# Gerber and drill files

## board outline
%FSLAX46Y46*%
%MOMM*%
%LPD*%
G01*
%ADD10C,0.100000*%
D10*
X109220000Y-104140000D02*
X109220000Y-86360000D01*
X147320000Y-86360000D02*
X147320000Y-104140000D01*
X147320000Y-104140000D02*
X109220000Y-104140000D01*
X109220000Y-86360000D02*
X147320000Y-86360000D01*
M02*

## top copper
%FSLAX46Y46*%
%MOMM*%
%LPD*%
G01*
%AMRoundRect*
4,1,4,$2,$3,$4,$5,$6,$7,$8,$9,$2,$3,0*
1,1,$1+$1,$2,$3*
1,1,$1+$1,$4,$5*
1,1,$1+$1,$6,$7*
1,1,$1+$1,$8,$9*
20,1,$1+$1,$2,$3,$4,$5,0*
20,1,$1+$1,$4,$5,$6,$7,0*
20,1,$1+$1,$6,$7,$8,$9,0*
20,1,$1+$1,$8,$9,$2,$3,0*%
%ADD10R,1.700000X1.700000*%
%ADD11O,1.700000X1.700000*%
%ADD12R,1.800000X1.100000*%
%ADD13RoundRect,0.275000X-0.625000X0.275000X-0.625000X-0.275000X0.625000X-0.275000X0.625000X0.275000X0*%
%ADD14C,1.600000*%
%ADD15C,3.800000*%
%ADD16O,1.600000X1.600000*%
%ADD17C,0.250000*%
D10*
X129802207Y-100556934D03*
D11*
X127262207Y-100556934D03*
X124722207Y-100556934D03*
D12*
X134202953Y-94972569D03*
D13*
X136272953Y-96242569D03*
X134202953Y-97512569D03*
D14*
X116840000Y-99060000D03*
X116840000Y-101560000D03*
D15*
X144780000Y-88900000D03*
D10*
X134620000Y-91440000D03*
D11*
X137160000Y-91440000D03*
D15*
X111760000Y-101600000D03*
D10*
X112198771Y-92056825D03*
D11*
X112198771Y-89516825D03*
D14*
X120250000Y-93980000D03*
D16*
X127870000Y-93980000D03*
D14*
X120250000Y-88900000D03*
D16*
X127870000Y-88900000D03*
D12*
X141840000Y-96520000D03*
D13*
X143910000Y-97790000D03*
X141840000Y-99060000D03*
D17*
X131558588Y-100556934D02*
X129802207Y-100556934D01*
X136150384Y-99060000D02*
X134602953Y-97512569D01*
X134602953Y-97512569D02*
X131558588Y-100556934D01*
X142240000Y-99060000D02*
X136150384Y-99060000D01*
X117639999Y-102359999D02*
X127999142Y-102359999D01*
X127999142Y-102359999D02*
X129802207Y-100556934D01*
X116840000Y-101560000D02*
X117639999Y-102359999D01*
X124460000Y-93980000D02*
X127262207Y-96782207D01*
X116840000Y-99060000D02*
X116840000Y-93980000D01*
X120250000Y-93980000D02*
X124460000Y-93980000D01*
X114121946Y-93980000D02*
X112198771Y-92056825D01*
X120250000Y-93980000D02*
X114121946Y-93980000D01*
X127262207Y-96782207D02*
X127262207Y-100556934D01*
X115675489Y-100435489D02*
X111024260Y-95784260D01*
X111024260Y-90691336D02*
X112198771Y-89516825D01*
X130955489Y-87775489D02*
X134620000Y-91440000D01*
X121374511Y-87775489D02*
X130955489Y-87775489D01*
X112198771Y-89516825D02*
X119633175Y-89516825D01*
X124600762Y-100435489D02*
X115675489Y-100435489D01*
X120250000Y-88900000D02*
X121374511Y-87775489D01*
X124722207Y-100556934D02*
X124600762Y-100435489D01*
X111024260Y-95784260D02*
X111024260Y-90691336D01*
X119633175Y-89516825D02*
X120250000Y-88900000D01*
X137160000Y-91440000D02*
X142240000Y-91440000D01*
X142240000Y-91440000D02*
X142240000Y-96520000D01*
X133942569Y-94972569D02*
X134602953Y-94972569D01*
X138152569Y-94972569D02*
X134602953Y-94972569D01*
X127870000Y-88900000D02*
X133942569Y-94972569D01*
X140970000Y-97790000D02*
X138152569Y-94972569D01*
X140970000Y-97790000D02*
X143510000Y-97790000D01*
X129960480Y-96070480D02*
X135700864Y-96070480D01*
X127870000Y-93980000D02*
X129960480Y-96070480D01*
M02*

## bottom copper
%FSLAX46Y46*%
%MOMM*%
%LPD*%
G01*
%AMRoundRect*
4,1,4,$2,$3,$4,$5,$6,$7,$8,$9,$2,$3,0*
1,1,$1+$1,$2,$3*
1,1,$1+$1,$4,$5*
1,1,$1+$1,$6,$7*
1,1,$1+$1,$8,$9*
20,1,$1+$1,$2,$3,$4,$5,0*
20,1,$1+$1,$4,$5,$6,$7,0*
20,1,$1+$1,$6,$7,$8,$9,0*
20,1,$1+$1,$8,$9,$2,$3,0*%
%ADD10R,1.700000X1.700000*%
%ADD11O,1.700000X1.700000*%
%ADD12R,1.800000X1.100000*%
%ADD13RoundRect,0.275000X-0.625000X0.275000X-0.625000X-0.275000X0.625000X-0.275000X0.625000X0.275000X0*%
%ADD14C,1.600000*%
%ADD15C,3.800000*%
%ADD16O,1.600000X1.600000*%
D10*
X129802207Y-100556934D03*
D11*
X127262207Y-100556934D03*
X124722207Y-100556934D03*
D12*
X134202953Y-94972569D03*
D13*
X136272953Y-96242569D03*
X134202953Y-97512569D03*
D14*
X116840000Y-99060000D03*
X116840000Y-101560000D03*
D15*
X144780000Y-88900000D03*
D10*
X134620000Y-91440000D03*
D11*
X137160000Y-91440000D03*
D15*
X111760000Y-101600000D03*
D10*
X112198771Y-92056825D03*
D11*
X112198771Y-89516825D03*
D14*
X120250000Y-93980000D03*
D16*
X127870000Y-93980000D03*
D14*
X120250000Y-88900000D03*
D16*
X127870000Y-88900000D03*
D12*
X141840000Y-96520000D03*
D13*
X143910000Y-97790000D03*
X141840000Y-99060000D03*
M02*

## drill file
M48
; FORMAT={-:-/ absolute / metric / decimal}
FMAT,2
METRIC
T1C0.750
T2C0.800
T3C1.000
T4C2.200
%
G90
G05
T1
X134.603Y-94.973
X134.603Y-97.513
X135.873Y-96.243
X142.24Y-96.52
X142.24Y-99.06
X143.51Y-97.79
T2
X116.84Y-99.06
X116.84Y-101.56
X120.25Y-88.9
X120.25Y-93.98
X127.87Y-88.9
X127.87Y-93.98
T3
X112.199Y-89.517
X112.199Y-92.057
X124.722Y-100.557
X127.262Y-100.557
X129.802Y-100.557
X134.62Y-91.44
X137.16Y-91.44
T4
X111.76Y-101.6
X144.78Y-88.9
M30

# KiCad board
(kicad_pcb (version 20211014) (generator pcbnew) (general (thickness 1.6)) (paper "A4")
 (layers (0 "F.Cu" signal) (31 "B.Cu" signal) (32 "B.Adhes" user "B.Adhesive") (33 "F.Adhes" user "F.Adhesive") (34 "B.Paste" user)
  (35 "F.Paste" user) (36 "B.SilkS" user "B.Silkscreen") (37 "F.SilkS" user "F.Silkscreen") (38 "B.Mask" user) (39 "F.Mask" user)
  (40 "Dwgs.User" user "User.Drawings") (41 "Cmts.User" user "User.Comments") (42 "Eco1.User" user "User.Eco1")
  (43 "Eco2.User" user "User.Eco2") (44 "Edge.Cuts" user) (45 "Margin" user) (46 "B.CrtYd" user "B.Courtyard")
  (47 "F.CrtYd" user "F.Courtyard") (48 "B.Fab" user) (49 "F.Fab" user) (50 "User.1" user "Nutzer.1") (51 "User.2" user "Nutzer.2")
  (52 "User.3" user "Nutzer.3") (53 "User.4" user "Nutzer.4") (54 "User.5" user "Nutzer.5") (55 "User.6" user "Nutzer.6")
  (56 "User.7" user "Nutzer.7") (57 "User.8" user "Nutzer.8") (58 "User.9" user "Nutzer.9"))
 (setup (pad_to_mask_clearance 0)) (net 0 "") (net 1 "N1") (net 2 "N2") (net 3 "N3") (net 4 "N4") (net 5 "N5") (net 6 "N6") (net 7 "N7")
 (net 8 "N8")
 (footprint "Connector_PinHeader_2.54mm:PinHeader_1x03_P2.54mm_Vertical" (layer "F.Cu") (at 129.802207 100.556934 -90)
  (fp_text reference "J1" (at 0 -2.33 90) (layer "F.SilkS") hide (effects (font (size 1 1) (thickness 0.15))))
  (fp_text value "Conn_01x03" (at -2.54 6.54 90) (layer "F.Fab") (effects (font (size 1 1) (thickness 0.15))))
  (pad "1" thru_hole rect (at 0 0 270) (size 1.7 1.7) (drill 1) (layers *.Cu *.Mask) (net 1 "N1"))
  (pad "2" thru_hole oval (at 0 2.54 270) (size 1.7 1.7) (drill 1) (layers *.Cu *.Mask) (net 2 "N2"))
  (pad "3" thru_hole oval (at 0 5.08 270) (size 1.7 1.7) (drill 1) (layers *.Cu *.Mask) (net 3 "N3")))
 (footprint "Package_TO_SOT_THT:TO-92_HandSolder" (layer "F.Cu") (at 134.602953 94.972569 -90)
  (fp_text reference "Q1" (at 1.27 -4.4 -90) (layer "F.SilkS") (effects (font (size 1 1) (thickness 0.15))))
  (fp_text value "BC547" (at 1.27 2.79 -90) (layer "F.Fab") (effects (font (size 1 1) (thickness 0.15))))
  (pad "1" thru_hole rect (at 0 0 270) (size 1.1 1.8) (drill 0.75 (offset 0 0.4)) (layers *.Cu *.Mask) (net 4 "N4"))
  (pad "2" thru_hole roundrect (at 1.27 -1.27 270) (size 1.1 1.8) (drill 0.75 (offset 0 -0.4)) (layers *.Cu *.Mask) (roundrect_rratio 0.25)
   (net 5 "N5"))
  (pad "3" thru_hole roundrect (at 2.54 0 270) (size 1.1 1.8) (drill 0.75 (offset 0 0.4)) (layers *.Cu *.Mask) (roundrect_rratio 0.25)
   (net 1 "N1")))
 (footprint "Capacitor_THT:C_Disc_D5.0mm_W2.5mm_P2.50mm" (layer "F.Cu") (at 116.84 99.06 -90)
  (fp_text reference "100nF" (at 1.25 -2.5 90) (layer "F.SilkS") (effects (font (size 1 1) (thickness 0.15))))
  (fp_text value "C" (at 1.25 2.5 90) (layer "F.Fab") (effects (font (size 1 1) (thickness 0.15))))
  (pad "1" thru_hole circle (at 0 0 270) (size 1.6 1.6) (drill 0.8) (layers *.Cu *.Mask) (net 2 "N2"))
  (pad "2" thru_hole circle (at 2.5 0 270) (size 1.6 1.6) (drill 0.8) (layers *.Cu *.Mask) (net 1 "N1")))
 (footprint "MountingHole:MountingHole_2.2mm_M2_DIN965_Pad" (layer "F.Cu") (at 144.78 88.9)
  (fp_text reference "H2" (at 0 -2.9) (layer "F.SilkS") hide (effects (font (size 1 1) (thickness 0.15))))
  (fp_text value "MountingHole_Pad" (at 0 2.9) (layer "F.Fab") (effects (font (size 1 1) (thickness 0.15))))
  (pad "1" thru_hole circle (at 0 0) (size 3.8 3.8) (drill 2.2) (layers *.Cu *.Mask) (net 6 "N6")))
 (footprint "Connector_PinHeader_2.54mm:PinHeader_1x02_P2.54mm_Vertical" (layer "F.Cu") (at 134.62 91.44 90)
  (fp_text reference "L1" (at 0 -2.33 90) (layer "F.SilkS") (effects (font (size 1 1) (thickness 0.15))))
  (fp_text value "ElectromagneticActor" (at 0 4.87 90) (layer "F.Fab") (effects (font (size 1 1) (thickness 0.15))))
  (pad "1" thru_hole rect (at 0 0 90) (size 1.7 1.7) (drill 1) (layers *.Cu *.Mask) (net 3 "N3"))
  (pad "2" thru_hole oval (at 0 2.54 90) (size 1.7 1.7) (drill 1) (layers *.Cu *.Mask) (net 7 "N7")))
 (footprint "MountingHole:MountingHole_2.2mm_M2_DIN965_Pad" (layer "F.Cu") (at 111.76 101.6)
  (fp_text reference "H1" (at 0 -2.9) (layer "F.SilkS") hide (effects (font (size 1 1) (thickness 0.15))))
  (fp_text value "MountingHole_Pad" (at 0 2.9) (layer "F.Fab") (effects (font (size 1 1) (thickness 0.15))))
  (pad "1" thru_hole circle (at 0 0) (size 3.8 3.8) (drill 2.2) (layers *.Cu *.Mask) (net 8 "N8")))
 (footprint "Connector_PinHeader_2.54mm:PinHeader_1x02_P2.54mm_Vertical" (layer "F.Cu") (at 112.198771 92.056825 180)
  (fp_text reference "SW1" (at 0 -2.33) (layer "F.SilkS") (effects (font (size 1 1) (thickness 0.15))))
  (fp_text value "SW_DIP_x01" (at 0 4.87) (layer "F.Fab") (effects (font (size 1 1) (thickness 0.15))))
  (pad "1" thru_hole rect (at 0 0 180) (size 1.7 1.7) (drill 1) (layers *.Cu *.Mask) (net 2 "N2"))
  (pad "2" thru_hole oval (at 0 2.54 180) (size 1.7 1.7) (drill 1) (layers *.Cu *.Mask) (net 3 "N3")))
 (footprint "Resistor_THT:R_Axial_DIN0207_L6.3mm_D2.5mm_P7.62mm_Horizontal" (layer "F.Cu") (at 120.25 93.98)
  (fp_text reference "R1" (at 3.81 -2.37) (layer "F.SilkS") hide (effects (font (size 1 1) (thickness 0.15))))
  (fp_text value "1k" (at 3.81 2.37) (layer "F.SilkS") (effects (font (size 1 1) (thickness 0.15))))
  (pad "1" thru_hole circle (at 0 0) (size 1.6 1.6) (drill 0.8) (layers *.Cu *.Mask) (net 2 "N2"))
  (pad "2" thru_hole oval (at 7.62 0) (size 1.6 1.6) (drill 0.8) (layers *.Cu *.Mask) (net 5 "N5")))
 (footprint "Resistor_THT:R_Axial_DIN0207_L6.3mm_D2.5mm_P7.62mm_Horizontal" (layer "F.Cu") (at 120.25 88.9)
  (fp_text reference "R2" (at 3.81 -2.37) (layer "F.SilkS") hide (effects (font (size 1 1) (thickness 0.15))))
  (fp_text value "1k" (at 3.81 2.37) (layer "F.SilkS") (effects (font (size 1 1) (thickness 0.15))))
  (pad "1" thru_hole circle (at 0 0) (size 1.6 1.6) (drill 0.8) (layers *.Cu *.Mask) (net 3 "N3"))
  (pad "2" thru_hole oval (at 7.62 0) (size 1.6 1.6) (drill 0.8) (layers *.Cu *.Mask) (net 4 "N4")))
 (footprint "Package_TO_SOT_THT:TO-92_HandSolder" (layer "F.Cu") (at 142.24 96.52 -90)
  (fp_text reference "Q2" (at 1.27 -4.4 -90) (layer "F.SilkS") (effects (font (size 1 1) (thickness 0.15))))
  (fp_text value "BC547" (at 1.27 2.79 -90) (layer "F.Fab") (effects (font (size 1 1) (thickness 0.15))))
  (pad "1" thru_hole rect (at 0 0 270) (size 1.1 1.8) (drill 0.75 (offset 0 0.4)) (layers *.Cu *.Mask) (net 7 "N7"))
  (pad "2" thru_hole roundrect (at 1.27 -1.27 270) (size 1.1 1.8) (drill 0.75 (offset 0 -0.4)) (layers *.Cu *.Mask) (roundrect_rratio 0.25)
   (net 4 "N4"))
  (pad "3" thru_hole roundrect (at 2.54 0 270) (size 1.1 1.8) (drill 0.75 (offset 0 0.4)) (layers *.Cu *.Mask) (roundrect_rratio 0.25)
   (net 1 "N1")))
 (gr_line (start 109.22 104.14) (end 109.22 86.36) (layer "Edge.Cuts") (width 0.1))
 (gr_line (start 147.32 86.36) (end 147.32 104.14) (layer "Edge.Cuts") (width 0.1))
 (gr_line (start 147.32 104.14) (end 109.22 104.14) (layer "Edge.Cuts") (width 0.1))
 (gr_line (start 109.22 86.36) (end 147.32 86.36) (layer "Edge.Cuts") (width 0.1))
 (segment (start 131.558588 100.556934) (end 129.802207 100.556934) (width 0.25) (layer "F.Cu") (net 1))
 (segment (start 136.150384 99.06) (end 134.602953 97.512569) (width 0.25) (layer "F.Cu") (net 1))
 (segment (start 134.602953 97.512569) (end 131.558588 100.556934) (width 0.25) (layer "F.Cu") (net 1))
 (segment (start 142.24 99.06) (end 136.150384 99.06) (width 0.25) (layer "F.Cu") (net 1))
 (segment (start 117.639999 102.359999) (end 127.999142 102.359999) (width 0.25) (layer "F.Cu") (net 1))
 (segment (start 127.999142 102.359999) (end 129.802207 100.556934) (width 0.25) (layer "F.Cu") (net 1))
 (segment (start 116.84 101.56) (end 117.639999 102.359999) (width 0.25) (layer "F.Cu") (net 1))
 (segment (start 124.46 93.98) (end 127.262207 96.782207) (width 0.25) (layer "F.Cu") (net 2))
 (segment (start 116.84 99.06) (end 116.84 93.98) (width 0.25) (layer "F.Cu") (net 2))
 (segment (start 120.25 93.98) (end 124.46 93.98) (width 0.25) (layer "F.Cu") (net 2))
 (segment (start 114.121946 93.98) (end 112.198771 92.056825) (width 0.25) (layer "F.Cu") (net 2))
 (segment (start 120.25 93.98) (end 114.121946 93.98) (width 0.25) (layer "F.Cu") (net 2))
 (segment (start 127.262207 96.782207) (end 127.262207 100.556934) (width 0.25) (layer "F.Cu") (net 2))
 (segment (start 115.675489 100.435489) (end 111.02426 95.78426) (width 0.25) (layer "F.Cu") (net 3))
 (segment (start 111.02426 90.691336) (end 112.198771 89.516825) (width 0.25) (layer "F.Cu") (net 3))
 (segment (start 130.955489 87.775489) (end 134.62 91.44) (width 0.25) (layer "F.Cu") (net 3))
 (segment (start 121.374511 87.775489) (end 130.955489 87.775489) (width 0.25) (layer "F.Cu") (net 3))
 (segment (start 112.198771 89.516825) (end 119.633175 89.516825) (width 0.25) (layer "F.Cu") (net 3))
 (segment (start 124.600762 100.435489) (end 115.675489 100.435489) (width 0.25) (layer "F.Cu") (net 3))
 (segment (start 120.25 88.9) (end 121.374511 87.775489) (width 0.25) (layer "F.Cu") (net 3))
 (segment (start 124.722207 100.556934) (end 124.600762 100.435489) (width 0.25) (layer "F.Cu") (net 3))
 (segment (start 111.02426 95.78426) (end 111.02426 90.691336) (width 0.25) (layer "F.Cu") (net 3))
 (segment (start 119.633175 89.516825) (end 120.25 88.9) (width 0.25) (layer "F.Cu") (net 3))
 (segment (start 137.16 91.44) (end 142.24 91.44) (width 0.25) (layer "F.Cu") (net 7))
 (segment (start 142.24 91.44) (end 142.24 96.52) (width 0.25) (layer "F.Cu") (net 7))
 (segment (start 133.942569 94.972569) (end 134.602953 94.972569) (width 0.25) (layer "F.Cu") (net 4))
 (segment (start 138.152569 94.972569) (end 134.602953 94.972569) (width 0.25) (layer "F.Cu") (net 4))
 (segment (start 127.87 88.9) (end 133.942569 94.972569) (width 0.25) (layer "F.Cu") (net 4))
 (segment (start 140.97 97.79) (end 138.152569 94.972569) (width 0.25) (layer "F.Cu") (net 4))
 (segment (start 140.97 97.79) (end 143.51 97.79) (width 0.25) (layer "F.Cu") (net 4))
 (segment (start 129.96048 96.07048) (end 135.700864 96.07048) (width 0.25) (layer "F.Cu") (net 5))
 (segment (start 127.87 93.98) (end 129.96048 96.07048) (width 0.25) (layer "F.Cu") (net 5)))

